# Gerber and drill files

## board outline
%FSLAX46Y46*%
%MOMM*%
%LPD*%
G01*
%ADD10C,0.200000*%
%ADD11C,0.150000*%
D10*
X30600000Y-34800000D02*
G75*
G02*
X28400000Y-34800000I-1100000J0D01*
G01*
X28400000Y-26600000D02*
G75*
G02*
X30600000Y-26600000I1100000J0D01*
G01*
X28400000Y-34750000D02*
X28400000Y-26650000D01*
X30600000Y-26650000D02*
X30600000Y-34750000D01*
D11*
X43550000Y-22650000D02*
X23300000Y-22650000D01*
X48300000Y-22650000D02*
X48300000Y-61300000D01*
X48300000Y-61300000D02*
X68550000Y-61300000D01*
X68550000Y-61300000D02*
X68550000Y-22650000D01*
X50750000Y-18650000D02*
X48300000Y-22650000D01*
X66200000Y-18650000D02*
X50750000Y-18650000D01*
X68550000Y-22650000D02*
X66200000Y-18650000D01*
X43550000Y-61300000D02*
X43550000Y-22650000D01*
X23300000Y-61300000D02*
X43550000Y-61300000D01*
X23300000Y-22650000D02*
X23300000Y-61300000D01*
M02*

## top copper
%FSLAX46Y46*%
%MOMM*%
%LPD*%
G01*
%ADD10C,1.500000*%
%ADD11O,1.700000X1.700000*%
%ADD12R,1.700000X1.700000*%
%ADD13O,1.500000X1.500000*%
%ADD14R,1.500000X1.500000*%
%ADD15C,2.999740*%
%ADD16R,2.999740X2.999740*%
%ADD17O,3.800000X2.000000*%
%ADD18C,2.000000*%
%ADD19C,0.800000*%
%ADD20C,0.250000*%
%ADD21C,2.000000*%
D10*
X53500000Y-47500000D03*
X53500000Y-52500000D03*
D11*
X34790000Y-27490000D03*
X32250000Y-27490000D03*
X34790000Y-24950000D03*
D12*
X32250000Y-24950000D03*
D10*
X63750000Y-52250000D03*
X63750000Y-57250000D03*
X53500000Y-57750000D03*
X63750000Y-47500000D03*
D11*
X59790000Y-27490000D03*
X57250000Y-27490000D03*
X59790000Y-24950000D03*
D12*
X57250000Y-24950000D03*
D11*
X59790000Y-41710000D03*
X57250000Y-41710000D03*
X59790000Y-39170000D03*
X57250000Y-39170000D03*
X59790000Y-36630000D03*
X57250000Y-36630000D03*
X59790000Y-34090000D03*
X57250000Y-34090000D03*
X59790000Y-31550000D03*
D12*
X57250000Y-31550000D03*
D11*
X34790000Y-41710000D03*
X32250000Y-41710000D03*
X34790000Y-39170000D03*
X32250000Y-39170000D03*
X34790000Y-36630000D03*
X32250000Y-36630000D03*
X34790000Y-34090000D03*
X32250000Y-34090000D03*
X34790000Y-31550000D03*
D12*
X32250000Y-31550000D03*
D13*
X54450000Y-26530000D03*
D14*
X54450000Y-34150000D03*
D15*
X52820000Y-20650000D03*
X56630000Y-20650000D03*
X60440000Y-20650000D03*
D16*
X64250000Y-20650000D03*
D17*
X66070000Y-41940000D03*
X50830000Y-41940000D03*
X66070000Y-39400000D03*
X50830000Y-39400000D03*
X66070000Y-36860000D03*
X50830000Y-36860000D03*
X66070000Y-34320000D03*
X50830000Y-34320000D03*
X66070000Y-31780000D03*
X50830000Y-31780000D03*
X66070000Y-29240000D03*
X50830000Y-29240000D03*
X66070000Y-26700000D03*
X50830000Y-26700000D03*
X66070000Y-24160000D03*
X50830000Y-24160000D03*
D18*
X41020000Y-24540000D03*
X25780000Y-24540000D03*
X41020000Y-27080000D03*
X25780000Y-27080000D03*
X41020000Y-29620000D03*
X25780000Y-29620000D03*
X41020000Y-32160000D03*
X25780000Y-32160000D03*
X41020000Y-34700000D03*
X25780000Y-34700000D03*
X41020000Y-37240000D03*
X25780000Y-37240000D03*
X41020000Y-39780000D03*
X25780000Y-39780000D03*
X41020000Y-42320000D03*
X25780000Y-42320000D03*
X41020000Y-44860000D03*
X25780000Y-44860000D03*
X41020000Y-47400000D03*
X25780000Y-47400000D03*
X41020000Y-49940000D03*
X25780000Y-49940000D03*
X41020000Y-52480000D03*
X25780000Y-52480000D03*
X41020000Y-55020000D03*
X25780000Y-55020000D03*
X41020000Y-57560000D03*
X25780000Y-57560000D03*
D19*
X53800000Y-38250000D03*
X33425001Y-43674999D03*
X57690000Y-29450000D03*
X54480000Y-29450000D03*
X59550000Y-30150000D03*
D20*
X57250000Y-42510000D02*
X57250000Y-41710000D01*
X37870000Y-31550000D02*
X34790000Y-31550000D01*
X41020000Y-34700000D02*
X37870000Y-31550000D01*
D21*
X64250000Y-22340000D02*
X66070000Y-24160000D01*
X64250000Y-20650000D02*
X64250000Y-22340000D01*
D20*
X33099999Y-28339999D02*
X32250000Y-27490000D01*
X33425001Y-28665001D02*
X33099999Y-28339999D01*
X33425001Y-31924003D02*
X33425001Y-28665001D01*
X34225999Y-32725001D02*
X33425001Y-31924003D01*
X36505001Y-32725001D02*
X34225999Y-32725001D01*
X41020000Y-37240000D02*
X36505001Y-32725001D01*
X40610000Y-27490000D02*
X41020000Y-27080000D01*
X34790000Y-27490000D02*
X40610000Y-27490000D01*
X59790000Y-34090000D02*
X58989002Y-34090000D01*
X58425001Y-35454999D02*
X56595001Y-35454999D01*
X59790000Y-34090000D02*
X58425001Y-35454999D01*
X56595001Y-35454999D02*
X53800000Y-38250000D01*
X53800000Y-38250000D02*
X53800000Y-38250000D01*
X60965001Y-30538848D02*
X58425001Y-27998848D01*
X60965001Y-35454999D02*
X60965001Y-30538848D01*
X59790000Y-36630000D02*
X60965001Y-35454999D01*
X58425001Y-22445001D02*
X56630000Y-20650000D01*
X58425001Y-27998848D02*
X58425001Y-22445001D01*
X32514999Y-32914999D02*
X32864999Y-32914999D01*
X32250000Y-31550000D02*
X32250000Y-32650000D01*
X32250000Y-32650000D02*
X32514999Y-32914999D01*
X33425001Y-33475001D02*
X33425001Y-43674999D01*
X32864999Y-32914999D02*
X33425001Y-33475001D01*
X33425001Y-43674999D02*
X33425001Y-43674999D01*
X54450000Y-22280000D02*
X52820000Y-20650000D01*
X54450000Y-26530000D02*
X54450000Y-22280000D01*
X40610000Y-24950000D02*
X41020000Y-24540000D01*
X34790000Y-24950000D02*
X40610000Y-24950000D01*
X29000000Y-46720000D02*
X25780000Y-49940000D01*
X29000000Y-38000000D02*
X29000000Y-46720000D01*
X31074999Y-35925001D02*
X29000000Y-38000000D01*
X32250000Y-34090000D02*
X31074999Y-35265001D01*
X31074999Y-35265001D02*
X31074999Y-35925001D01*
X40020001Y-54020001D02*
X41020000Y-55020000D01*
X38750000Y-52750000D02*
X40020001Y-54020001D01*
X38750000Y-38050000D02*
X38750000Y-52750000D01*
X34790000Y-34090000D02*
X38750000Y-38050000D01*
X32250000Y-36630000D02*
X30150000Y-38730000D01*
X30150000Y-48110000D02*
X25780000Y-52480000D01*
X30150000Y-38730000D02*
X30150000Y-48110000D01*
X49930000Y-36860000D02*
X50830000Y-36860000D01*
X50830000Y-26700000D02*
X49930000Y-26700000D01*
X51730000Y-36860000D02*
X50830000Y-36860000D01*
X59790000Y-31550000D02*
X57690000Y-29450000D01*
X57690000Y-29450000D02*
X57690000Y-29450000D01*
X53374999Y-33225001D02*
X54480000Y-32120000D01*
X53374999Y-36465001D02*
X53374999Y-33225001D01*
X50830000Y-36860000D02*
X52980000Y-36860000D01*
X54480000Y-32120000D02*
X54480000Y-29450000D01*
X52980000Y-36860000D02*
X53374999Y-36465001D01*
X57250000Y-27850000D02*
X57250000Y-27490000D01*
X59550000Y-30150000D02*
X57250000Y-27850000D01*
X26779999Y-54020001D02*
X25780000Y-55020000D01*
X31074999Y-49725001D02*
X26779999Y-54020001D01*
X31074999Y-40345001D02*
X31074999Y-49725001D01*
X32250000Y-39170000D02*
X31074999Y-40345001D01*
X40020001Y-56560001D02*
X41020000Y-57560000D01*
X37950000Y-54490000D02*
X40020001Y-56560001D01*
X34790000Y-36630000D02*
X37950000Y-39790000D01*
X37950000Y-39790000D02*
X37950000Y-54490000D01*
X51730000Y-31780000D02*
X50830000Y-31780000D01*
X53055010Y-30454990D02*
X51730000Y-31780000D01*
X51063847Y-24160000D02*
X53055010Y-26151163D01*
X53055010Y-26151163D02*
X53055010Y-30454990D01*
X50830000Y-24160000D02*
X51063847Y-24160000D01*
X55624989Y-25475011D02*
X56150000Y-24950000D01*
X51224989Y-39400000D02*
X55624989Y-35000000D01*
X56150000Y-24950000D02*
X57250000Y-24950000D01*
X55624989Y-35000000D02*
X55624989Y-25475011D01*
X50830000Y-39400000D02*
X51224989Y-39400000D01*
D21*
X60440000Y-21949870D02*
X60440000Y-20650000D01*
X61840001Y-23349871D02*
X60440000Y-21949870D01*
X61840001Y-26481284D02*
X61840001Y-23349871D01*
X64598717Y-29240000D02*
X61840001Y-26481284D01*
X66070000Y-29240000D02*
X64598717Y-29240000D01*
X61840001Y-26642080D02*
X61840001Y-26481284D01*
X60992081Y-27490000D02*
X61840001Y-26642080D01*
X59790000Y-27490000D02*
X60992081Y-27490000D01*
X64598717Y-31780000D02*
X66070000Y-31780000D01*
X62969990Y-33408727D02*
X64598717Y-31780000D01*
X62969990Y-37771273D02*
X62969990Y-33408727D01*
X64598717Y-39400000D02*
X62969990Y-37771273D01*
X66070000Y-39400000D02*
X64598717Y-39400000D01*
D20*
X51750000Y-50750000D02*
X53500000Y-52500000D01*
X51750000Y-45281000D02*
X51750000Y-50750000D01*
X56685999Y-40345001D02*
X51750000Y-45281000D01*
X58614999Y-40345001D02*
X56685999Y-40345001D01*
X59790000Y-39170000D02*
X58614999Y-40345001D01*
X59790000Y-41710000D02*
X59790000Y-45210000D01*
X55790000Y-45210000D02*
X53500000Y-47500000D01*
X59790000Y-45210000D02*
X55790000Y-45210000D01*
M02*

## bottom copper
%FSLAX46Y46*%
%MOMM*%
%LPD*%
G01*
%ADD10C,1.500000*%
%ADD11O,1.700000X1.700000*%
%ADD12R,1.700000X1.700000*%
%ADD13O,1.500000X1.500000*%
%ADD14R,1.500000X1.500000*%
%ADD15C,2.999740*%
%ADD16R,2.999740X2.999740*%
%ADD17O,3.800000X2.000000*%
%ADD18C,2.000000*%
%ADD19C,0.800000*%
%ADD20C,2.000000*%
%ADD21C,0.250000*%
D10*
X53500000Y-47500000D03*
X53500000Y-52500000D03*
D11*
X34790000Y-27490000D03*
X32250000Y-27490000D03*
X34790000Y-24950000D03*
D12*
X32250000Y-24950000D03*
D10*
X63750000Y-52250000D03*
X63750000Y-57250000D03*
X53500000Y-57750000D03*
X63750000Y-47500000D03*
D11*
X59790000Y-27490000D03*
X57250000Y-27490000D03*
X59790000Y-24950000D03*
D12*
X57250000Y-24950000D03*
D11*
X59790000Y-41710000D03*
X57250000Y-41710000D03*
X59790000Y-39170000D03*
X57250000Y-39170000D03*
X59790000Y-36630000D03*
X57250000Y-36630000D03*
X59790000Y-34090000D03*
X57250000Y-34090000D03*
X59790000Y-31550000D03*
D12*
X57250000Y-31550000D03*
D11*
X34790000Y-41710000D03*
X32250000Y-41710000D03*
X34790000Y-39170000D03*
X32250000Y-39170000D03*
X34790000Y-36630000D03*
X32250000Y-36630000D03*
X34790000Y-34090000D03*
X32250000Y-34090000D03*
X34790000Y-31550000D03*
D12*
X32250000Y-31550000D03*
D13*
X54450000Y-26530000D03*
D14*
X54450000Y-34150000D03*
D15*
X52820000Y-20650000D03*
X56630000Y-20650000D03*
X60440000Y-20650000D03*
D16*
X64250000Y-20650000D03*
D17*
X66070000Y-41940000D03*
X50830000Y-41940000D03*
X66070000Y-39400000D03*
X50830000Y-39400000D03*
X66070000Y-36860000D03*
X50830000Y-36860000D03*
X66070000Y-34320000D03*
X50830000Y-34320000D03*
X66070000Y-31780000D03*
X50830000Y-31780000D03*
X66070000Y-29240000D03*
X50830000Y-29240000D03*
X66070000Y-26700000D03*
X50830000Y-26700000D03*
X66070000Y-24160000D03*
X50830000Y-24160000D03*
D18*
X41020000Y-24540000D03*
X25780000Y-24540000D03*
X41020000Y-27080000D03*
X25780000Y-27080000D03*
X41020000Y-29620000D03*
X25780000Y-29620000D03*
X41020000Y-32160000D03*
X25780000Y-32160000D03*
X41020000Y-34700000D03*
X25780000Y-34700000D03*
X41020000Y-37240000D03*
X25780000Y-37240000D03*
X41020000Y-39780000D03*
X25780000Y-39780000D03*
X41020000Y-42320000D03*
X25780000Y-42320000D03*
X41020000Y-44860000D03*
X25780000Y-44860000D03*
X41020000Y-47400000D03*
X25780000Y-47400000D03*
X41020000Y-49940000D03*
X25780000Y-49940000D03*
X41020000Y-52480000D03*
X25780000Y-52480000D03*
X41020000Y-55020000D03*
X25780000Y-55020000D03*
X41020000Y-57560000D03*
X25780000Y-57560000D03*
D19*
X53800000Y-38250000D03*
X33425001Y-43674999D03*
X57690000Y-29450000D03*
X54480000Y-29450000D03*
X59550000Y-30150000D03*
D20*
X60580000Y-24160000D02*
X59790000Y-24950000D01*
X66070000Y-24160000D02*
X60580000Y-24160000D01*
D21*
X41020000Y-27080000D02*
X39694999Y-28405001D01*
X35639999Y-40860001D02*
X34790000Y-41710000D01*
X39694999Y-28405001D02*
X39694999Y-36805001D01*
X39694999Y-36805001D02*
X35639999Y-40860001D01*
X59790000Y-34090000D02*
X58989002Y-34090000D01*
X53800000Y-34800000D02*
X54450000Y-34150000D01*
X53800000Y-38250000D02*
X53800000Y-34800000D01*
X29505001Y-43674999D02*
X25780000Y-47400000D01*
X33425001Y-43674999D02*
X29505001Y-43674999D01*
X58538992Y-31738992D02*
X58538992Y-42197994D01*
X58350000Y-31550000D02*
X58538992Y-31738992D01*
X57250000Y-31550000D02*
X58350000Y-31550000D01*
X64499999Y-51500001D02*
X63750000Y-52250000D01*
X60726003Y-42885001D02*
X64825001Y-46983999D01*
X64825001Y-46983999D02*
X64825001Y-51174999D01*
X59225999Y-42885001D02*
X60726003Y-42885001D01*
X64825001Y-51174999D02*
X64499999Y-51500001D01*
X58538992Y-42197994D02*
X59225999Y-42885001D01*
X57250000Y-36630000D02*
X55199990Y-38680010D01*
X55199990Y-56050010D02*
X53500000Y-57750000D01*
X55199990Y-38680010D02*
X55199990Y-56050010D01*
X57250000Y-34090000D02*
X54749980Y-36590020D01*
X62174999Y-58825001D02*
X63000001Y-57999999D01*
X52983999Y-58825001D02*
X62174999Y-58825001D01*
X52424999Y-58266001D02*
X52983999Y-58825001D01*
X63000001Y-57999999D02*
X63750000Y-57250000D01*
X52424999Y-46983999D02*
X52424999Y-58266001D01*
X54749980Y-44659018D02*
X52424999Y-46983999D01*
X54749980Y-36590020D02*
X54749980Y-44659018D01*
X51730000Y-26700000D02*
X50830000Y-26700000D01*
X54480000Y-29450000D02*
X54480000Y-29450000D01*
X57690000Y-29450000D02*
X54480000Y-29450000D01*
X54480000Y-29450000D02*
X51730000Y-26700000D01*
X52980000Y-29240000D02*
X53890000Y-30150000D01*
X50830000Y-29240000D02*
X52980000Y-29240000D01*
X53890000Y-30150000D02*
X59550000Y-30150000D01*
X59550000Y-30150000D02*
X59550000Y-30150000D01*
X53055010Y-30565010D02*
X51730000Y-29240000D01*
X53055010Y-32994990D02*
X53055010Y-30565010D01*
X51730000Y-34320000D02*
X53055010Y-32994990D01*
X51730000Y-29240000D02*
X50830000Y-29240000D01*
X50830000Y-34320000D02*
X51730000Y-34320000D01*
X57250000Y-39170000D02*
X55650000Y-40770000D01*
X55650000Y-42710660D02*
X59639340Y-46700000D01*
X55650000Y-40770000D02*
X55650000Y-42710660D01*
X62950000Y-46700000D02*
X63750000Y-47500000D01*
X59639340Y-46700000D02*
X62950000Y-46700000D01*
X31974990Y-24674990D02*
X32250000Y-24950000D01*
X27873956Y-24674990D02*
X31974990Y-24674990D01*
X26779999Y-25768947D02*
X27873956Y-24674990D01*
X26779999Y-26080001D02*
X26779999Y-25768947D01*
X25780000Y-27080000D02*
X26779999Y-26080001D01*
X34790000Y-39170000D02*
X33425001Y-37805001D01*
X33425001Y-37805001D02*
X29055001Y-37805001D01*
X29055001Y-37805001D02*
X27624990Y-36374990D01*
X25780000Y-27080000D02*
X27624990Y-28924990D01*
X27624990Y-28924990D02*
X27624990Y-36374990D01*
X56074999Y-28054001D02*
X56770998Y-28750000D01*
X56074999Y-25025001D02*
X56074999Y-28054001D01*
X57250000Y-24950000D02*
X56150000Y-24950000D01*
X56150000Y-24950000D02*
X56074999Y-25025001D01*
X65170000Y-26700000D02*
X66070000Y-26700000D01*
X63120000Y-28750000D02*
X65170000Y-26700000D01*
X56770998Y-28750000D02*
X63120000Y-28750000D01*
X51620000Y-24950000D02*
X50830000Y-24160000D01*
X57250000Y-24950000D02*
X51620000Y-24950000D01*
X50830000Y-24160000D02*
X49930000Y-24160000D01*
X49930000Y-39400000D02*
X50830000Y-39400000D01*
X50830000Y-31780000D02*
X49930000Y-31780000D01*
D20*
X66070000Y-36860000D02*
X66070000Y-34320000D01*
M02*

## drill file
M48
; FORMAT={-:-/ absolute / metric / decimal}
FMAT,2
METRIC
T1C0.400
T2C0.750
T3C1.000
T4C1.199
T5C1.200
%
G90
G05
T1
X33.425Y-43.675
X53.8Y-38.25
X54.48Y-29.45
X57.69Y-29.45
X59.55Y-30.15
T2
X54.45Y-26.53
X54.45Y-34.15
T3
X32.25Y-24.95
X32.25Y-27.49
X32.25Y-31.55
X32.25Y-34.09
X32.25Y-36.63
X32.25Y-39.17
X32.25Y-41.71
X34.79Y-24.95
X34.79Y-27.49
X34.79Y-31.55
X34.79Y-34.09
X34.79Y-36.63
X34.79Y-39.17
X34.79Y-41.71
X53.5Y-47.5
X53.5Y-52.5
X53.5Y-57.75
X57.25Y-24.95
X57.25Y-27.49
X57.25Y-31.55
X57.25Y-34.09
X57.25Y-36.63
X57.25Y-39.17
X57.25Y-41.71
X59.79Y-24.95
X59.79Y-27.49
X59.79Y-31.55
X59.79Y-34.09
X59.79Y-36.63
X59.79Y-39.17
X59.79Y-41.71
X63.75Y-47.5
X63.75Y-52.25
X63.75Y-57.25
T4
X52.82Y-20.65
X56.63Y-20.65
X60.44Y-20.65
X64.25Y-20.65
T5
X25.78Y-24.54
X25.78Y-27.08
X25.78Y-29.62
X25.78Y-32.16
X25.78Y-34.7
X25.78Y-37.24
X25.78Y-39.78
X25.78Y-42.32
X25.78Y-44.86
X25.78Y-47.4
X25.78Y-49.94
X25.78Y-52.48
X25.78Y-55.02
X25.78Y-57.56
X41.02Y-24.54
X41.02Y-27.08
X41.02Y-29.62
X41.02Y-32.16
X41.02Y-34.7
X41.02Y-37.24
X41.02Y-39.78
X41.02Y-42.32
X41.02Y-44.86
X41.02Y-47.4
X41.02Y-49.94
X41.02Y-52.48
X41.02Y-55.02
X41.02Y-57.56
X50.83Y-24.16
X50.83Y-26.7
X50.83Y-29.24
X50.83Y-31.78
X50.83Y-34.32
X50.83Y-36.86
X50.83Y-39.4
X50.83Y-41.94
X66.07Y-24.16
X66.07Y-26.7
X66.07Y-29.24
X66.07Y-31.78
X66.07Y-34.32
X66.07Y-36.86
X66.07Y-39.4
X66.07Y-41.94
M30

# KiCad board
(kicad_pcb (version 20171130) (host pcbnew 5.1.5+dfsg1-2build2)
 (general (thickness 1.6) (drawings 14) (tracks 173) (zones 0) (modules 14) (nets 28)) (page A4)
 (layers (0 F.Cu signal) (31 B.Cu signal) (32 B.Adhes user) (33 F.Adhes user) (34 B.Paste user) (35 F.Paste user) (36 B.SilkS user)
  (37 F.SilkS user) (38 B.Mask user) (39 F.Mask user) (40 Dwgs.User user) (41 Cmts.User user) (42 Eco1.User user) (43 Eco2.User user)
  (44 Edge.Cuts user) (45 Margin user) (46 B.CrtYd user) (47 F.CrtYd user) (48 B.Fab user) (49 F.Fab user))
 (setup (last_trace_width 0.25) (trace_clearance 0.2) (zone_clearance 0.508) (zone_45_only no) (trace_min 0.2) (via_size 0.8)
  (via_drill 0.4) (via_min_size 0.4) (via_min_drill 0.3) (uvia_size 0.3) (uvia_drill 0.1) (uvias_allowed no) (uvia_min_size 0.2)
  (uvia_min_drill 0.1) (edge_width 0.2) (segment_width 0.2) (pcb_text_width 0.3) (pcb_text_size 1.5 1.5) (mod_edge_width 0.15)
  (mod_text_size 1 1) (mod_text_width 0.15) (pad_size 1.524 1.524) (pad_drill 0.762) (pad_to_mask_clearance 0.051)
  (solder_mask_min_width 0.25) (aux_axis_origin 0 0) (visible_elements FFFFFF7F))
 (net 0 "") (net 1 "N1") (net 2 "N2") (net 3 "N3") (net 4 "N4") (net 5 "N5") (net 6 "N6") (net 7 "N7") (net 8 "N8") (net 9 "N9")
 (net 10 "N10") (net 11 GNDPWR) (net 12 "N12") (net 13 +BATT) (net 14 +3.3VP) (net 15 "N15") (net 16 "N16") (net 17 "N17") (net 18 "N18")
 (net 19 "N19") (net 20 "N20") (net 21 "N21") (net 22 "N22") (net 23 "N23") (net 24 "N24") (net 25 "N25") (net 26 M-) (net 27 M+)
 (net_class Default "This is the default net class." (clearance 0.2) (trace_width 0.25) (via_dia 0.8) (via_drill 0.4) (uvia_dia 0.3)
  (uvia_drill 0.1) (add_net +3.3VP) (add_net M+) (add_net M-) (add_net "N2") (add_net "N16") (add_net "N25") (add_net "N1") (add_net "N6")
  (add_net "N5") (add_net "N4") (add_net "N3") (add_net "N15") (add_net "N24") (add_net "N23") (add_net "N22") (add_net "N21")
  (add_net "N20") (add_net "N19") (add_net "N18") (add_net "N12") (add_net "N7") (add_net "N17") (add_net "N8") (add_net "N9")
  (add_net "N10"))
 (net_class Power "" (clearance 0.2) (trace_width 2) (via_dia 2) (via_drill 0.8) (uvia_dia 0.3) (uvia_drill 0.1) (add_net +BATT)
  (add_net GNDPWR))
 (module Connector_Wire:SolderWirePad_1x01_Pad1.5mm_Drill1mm (layer B.Cu) (at 53.5 47.5)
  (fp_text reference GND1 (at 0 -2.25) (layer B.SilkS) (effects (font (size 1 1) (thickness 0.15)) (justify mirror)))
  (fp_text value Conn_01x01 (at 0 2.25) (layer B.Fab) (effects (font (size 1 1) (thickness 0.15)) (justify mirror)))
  (pad 1 thru_hole circle (at 0 0) (size 1.5 1.5) (drill 1) (layers *.Cu *.Mask) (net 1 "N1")))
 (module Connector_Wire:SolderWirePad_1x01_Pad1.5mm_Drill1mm (layer B.Cu) (at 53.5 52.5)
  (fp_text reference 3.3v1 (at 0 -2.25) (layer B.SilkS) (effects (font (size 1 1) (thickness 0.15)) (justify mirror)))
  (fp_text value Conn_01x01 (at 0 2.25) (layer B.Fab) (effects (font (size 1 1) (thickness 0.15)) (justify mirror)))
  (pad 1 thru_hole circle (at 0 0) (size 1.5 1.5) (drill 1) (layers *.Cu *.Mask) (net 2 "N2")))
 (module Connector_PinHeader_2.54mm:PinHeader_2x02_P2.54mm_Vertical (layer F.Cu) (at 32.25 24.95)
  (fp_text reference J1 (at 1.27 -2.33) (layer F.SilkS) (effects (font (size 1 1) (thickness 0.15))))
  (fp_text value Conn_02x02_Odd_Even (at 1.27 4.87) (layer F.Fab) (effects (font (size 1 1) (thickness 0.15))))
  (pad 4 thru_hole oval (at 2.54 2.54) (size 1.7 1.7) (drill 1) (layers *.Cu *.Mask) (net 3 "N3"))
  (pad 3 thru_hole oval (at 0 2.54) (size 1.7 1.7) (drill 1) (layers *.Cu *.Mask) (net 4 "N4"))
  (pad 2 thru_hole oval (at 2.54 0) (size 1.7 1.7) (drill 1) (layers *.Cu *.Mask) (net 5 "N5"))
  (pad 1 thru_hole rect (at 0 0) (size 1.7 1.7) (drill 1) (layers *.Cu *.Mask) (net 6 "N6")))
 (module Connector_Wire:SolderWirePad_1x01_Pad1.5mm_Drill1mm (layer B.Cu) (at 63.75 52.25)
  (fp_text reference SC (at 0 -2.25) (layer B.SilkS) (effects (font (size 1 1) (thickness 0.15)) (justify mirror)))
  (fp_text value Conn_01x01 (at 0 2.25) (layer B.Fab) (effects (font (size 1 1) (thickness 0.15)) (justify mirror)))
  (pad 1 thru_hole circle (at 0 0) (size 1.5 1.5) (drill 1) (layers *.Cu *.Mask) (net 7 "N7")))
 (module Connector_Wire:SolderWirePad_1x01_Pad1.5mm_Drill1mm (layer B.Cu) (at 63.75 57.25)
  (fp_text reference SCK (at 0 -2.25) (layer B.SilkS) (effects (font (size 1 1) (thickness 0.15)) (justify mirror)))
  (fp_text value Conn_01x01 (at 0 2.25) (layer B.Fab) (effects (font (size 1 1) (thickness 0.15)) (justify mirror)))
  (pad 1 thru_hole circle (at 0 0) (size 1.5 1.5) (drill 1) (layers *.Cu *.Mask) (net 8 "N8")))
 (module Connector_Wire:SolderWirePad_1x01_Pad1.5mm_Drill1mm (layer B.Cu) (at 53.5 57.75)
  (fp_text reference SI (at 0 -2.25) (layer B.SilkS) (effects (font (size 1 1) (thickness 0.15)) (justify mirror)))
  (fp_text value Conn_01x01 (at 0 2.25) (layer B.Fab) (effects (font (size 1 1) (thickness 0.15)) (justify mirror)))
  (pad 1 thru_hole circle (at 0 0) (size 1.5 1.5) (drill 1) (layers *.Cu *.Mask) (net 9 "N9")))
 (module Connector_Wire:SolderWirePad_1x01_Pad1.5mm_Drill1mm (layer B.Cu) (at 63.75 47.5)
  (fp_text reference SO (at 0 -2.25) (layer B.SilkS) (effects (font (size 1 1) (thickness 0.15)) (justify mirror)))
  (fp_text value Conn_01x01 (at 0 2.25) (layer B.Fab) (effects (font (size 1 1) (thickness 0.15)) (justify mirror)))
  (pad 1 thru_hole circle (at 0 0) (size 1.5 1.5) (drill 1) (layers *.Cu *.Mask) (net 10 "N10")))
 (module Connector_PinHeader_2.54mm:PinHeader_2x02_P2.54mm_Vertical (layer F.Cu) (at 57.25 24.95)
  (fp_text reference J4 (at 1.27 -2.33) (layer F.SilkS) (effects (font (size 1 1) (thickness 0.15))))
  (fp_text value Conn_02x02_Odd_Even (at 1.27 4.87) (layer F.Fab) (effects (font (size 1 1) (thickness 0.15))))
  (pad 4 thru_hole oval (at 2.54 2.54) (size 1.7 1.7) (drill 1) (layers *.Cu *.Mask) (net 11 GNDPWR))
  (pad 3 thru_hole oval (at 0 2.54) (size 1.7 1.7) (drill 1) (layers *.Cu *.Mask) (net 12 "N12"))
  (pad 2 thru_hole oval (at 2.54 0) (size 1.7 1.7) (drill 1) (layers *.Cu *.Mask) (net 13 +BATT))
  (pad 1 thru_hole rect (at 0 0) (size 1.7 1.7) (drill 1) (layers *.Cu *.Mask) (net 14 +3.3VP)))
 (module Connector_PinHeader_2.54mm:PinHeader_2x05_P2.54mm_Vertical (layer F.Cu) (at 57.25 31.55)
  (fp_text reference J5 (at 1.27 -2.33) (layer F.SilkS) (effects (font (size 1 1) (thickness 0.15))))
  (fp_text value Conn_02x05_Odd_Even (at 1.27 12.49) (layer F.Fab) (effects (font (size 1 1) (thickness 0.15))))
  (pad 10 thru_hole oval (at 2.54 10.16) (size 1.7 1.7) (drill 1) (layers *.Cu *.Mask) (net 1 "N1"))
  (pad 9 thru_hole oval (at 0 10.16) (size 1.7 1.7) (drill 1) (layers *.Cu *.Mask))
  (pad 8 thru_hole oval (at 2.54 7.62) (size 1.7 1.7) (drill 1) (layers *.Cu *.Mask) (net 2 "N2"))
  (pad 7 thru_hole oval (at 0 7.62) (size 1.7 1.7) (drill 1) (layers *.Cu *.Mask) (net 10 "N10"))
  (pad 6 thru_hole oval (at 2.54 5.08) (size 1.7 1.7) (drill 1) (layers *.Cu *.Mask) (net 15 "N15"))
  (pad 5 thru_hole oval (at 0 5.08) (size 1.7 1.7) (drill 1) (layers *.Cu *.Mask) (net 9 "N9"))
  (pad 4 thru_hole oval (at 2.54 2.54) (size 1.7 1.7) (drill 1) (layers *.Cu *.Mask) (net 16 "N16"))
  (pad 3 thru_hole oval (at 0 2.54) (size 1.7 1.7) (drill 1) (layers *.Cu *.Mask) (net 8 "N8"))
  (pad 2 thru_hole oval (at 2.54 0) (size 1.7 1.7) (drill 1) (layers *.Cu *.Mask) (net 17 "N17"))
  (pad 1 thru_hole rect (at 0 0) (size 1.7 1.7) (drill 1) (layers *.Cu *.Mask) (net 7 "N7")))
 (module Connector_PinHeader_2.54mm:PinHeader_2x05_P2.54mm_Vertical (layer F.Cu) (at 32.25 31.55)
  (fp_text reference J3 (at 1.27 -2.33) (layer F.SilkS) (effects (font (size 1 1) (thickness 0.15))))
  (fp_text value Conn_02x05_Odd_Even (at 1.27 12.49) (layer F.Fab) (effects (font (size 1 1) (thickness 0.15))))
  (pad 10 thru_hole oval (at 2.54 10.16) (size 1.7 1.7) (drill 1) (layers *.Cu *.Mask) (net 3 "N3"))
  (pad 9 thru_hole oval (at 0 10.16) (size 1.7 1.7) (drill 1) (layers *.Cu *.Mask))
  (pad 8 thru_hole oval (at 2.54 7.62) (size 1.7 1.7) (drill 1) (layers *.Cu *.Mask) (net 6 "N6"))
  (pad 7 thru_hole oval (at 0 7.62) (size 1.7 1.7) (drill 1) (layers *.Cu *.Mask) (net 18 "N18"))
  (pad 6 thru_hole oval (at 2.54 5.08) (size 1.7 1.7) (drill 1) (layers *.Cu *.Mask) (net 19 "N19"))
  (pad 5 thru_hole oval (at 0 5.08) (size 1.7 1.7) (drill 1) (layers *.Cu *.Mask) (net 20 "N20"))
  (pad 4 thru_hole oval (at 2.54 2.54) (size 1.7 1.7) (drill 1) (layers *.Cu *.Mask) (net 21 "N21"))
  (pad 3 thru_hole oval (at 0 2.54) (size 1.7 1.7) (drill 1) (layers *.Cu *.Mask) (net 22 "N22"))
  (pad 2 thru_hole oval (at 2.54 0) (size 1.7 1.7) (drill 1) (layers *.Cu *.Mask) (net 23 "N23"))
  (pad 1 thru_hole rect (at 0 0) (size 1.7 1.7) (drill 1) (layers *.Cu *.Mask) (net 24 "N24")))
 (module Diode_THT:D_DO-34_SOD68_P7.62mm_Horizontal (layer F.Cu) (at 54.45 34.15 90)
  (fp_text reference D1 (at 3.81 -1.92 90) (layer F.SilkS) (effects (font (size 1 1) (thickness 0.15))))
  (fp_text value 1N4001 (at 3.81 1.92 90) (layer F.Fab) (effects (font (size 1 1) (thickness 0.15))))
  (pad 2 thru_hole oval (at 7.62 0 90) (size 1.5 1.5) (drill 0.75) (layers *.Cu *.Mask) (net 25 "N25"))
  (pad 1 thru_hole rect (at 0 0 90) (size 1.5 1.5) (drill 0.75) (layers *.Cu *.Mask) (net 16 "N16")))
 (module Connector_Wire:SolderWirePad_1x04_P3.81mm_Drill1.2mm (layer F.Cu) (at 64.25 20.65 180)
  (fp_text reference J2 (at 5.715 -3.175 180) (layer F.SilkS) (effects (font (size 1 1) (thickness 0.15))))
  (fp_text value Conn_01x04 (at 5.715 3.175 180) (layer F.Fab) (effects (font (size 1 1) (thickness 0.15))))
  (pad 4 thru_hole circle (at 11.43 0 180) (size 2.99974 2.99974) (drill 1.19888) (layers *.Cu *.Mask) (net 25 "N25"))
  (pad 3 thru_hole circle (at 7.62 0 180) (size 2.99974 2.99974) (drill 1.19888) (layers *.Cu *.Mask) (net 15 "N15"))
  (pad 2 thru_hole circle (at 3.81 0 180) (size 2.99974 2.99974) (drill 1.19888) (layers *.Cu *.Mask) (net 11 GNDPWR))
  (pad 1 thru_hole rect (at 0 0 180) (size 2.99974 2.99974) (drill 1.19888) (layers *.Cu *.Mask) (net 13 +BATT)))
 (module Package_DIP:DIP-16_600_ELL (layer B.Cu) (at 58.45 33.05 270)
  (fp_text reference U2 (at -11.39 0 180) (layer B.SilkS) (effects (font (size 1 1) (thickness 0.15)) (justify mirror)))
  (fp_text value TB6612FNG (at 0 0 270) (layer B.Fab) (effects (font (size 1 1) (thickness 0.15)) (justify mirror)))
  (pad 8 thru_hole oval (at 8.89 -7.62 270) (size 2 3.8) (drill 1.2) (layers *.Cu *.Mask))
  (pad 9 thru_hole oval (at 8.89 7.62 270) (size 2 3.8) (drill 1.2) (layers *.Cu *.Mask))
  (pad 7 thru_hole oval (at 6.35 -7.62 270) (size 2 3.8) (drill 1.2) (layers *.Cu *.Mask) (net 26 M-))
  (pad 10 thru_hole oval (at 6.35 7.62 270) (size 2 3.8) (drill 1.2) (layers *.Cu *.Mask) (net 14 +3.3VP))
  (pad 6 thru_hole oval (at 3.81 -7.62 270) (size 2 3.8) (drill 1.2) (layers *.Cu *.Mask) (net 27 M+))
  (pad 11 thru_hole oval (at 3.81 7.62 270) (size 2 3.8) (drill 1.2) (layers *.Cu *.Mask) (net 17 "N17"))
  (pad 5 thru_hole oval (at 1.27 -7.62 270) (size 2 3.8) (drill 1.2) (layers *.Cu *.Mask) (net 27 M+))
  (pad 12 thru_hole oval (at 1.27 7.62 270) (size 2 3.8) (drill 1.2) (layers *.Cu *.Mask) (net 12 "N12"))
  (pad 4 thru_hole oval (at -1.27 -7.62 270) (size 2 3.8) (drill 1.2) (layers *.Cu *.Mask) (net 26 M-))
  (pad 13 thru_hole oval (at -1.27 7.62 270) (size 2 3.8) (drill 1.2) (layers *.Cu *.Mask) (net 14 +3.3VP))
  (pad 3 thru_hole oval (at -3.81 -7.62 270) (size 2 3.8) (drill 1.2) (layers *.Cu *.Mask) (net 11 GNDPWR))
  (pad 14 thru_hole oval (at -3.81 7.62 270) (size 2 3.8) (drill 1.2) (layers *.Cu *.Mask) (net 12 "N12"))
  (pad 2 thru_hole oval (at -6.35 -7.62 270) (size 2 3.8) (drill 1.2) (layers *.Cu *.Mask) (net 14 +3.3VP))
  (pad 15 thru_hole oval (at -6.35 7.62 270) (size 2 3.8) (drill 1.2) (layers *.Cu *.Mask) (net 17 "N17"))
  (pad 1 thru_hole oval (at -8.89 -7.62 270) (size 2 3.8) (drill 1.2) (layers *.Cu *.Mask) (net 13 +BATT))
  (pad 16 thru_hole oval (at -8.89 7.62 270) (size 2 3.8) (drill 1.2) (layers *.Cu *.Mask) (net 14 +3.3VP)))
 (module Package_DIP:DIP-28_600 (layer F.Cu) (at 33.4 41.05 270)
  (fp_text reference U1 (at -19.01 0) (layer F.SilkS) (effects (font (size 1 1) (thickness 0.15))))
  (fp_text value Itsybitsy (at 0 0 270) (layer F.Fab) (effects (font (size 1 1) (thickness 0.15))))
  (pad 28 thru_hole circle (at -16.51 -7.62 270) (size 2 2) (drill 1.2) (layers *.Cu *.Mask) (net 5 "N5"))
  (pad 1 thru_hole circle (at -16.51 7.62 270) (size 2 2) (drill 1.2) (layers *.Cu *.Mask))
  (pad 27 thru_hole circle (at -13.97 -7.62 270) (size 2 2) (drill 1.2) (layers *.Cu *.Mask) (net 3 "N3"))
  (pad 2 thru_hole circle (at -13.97 7.62 270) (size 2 2) (drill 1.2) (layers *.Cu *.Mask) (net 6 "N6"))
  (pad 26 thru_hole circle (at -11.43 -7.62 270) (size 2 2) (drill 1.2) (layers *.Cu *.Mask))
  (pad 3 thru_hole circle (at -11.43 7.62 270) (size 2 2) (drill 1.2) (layers *.Cu *.Mask))
  (pad 25 thru_hole circle (at -8.89 -7.62 270) (size 2 2) (drill 1.2) (layers *.Cu *.Mask))
  (pad 4 thru_hole circle (at -8.89 7.62 270) (size 2 2) (drill 1.2) (layers *.Cu *.Mask))
  (pad 24 thru_hole circle (at -6.35 -7.62 270) (size 2 2) (drill 1.2) (layers *.Cu *.Mask) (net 23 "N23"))
  (pad 5 thru_hole circle (at -6.35 7.62 270) (size 2 2) (drill 1.2) (layers *.Cu *.Mask))
  (pad 23 thru_hole circle (at -3.81 -7.62 270) (size 2 2) (drill 1.2) (layers *.Cu *.Mask) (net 4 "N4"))
  (pad 6 thru_hole circle (at -3.81 7.62 270) (size 2 2) (drill 1.2) (layers *.Cu *.Mask))
  (pad 22 thru_hole circle (at -1.27 -7.62 270) (size 2 2) (drill 1.2) (layers *.Cu *.Mask))
  (pad 7 thru_hole circle (at -1.27 7.62 270) (size 2 2) (drill 1.2) (layers *.Cu *.Mask))
  (pad 21 thru_hole circle (at 1.27 -7.62 270) (size 2 2) (drill 1.2) (layers *.Cu *.Mask))
  (pad 8 thru_hole circle (at 1.27 7.62 270) (size 2 2) (drill 1.2) (layers *.Cu *.Mask))
  (pad 20 thru_hole circle (at 3.81 -7.62 270) (size 2 2) (drill 1.2) (layers *.Cu *.Mask))
  (pad 9 thru_hole circle (at 3.81 7.62 270) (size 2 2) (drill 1.2) (layers *.Cu *.Mask))
  (pad 19 thru_hole circle (at 6.35 -7.62 270) (size 2 2) (drill 1.2) (layers *.Cu *.Mask))
  (pad 10 thru_hole circle (at 6.35 7.62 270) (size 2 2) (drill 1.2) (layers *.Cu *.Mask) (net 24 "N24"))
  (pad 18 thru_hole circle (at 8.89 -7.62 270) (size 2 2) (drill 1.2) (layers *.Cu *.Mask))
  (pad 11 thru_hole circle (at 8.89 7.62 270) (size 2 2) (drill 1.2) (layers *.Cu *.Mask) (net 22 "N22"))
  (pad 17 thru_hole circle (at 11.43 -7.62 270) (size 2 2) (drill 1.2) (layers *.Cu *.Mask))
  (pad 12 thru_hole circle (at 11.43 7.62 270) (size 2 2) (drill 1.2) (layers *.Cu *.Mask) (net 20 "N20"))
  (pad 16 thru_hole circle (at 13.97 -7.62 270) (size 2 2) (drill 1.2) (layers *.Cu *.Mask) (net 21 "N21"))
  (pad 13 thru_hole circle (at 13.97 7.62 270) (size 2 2) (drill 1.2) (layers *.Cu *.Mask) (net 18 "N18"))
  (pad 15 thru_hole circle (at 16.51 -7.62 270) (size 2 2) (drill 1.2) (layers *.Cu *.Mask) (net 19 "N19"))
  (pad 14 thru_hole circle (at 16.51 7.62 270) (size 2 2) (drill 1.2) (layers *.Cu *.Mask)))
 (gr_arc (start 29.5 34.8) (end 28.4 34.8) (angle -180) (layer Edge.Cuts) (width 0.2))
 (gr_arc (start 29.5 26.6) (end 30.6 26.6) (angle -180) (layer Edge.Cuts) (width 0.2))
 (gr_line (start 28.4 34.75) (end 28.4 26.65) (layer Edge.Cuts) (width 0.2))
 (gr_line (start 30.6 26.65) (end 30.6 34.75) (layer Edge.Cuts) (width 0.2))
 (gr_line (start 43.55 22.65) (end 23.3 22.65) (layer Edge.Cuts) (width 0.15))
 (gr_line (start 48.3 22.65) (end 48.3 61.3) (layer Edge.Cuts) (width 0.15))
 (gr_line (start 48.3 61.3) (end 68.55 61.3) (layer Edge.Cuts) (width 0.15))
 (gr_line (start 68.55 61.3) (end 68.55 22.65) (layer Edge.Cuts) (width 0.15))
 (gr_line (start 50.75 18.65) (end 48.3 22.65) (layer Edge.Cuts) (width 0.15))
 (gr_line (start 66.2 18.65) (end 50.75 18.65) (layer Edge.Cuts) (width 0.15))
 (gr_line (start 68.55 22.65) (end 66.2 18.65) (layer Edge.Cuts) (width 0.15))
 (gr_line (start 43.55 61.3) (end 43.55 22.65) (layer Edge.Cuts) (width 0.15))
 (gr_line (start 23.3 61.3) (end 43.55 61.3) (layer Edge.Cuts) (width 0.15))
 (gr_line (start 23.3 22.65) (end 23.3 61.3) (layer Edge.Cuts) (width 0.15))
 (segment (start 57.25 42.51) (end 57.25 41.71) (width 0.25) (layer F.Cu) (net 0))
 (segment (start 37.87 31.55) (end 34.79 31.55) (width 0.25) (layer F.Cu) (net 23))
 (segment (start 41.02 34.7) (end 37.87 31.55) (width 0.25) (layer F.Cu) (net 23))
 (segment (start 60.58 24.16) (end 59.79 24.95) (width 2) (layer B.Cu) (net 13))
 (segment (start 66.07 24.16) (end 60.58 24.16) (width 2) (layer B.Cu) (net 13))
 (segment (start 64.25 22.34) (end 66.07 24.16) (width 2) (layer F.Cu) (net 13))
 (segment (start 64.25 20.65) (end 64.25 22.34) (width 2) (layer F.Cu) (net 13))
 (segment (start 33.099999 28.339999) (end 32.25 27.49) (width 0.25) (layer F.Cu) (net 4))
 (segment (start 33.425001 28.665001) (end 33.099999 28.339999) (width 0.25) (layer F.Cu) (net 4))
 (segment (start 33.425001 31.924003) (end 33.425001 28.665001) (width 0.25) (layer F.Cu) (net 4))
 (segment (start 34.225999 32.725001) (end 33.425001 31.924003) (width 0.25) (layer F.Cu) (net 4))
 (segment (start 36.505001 32.725001) (end 34.225999 32.725001) (width 0.25) (layer F.Cu) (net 4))
 (segment (start 41.02 37.24) (end 36.505001 32.725001) (width 0.25) (layer F.Cu) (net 4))
 (segment (start 40.61 27.49) (end 41.02 27.08) (width 0.25) (layer F.Cu) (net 3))
 (segment (start 34.79 27.49) (end 40.61 27.49) (width 0.25) (layer F.Cu) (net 3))
 (segment (start 41.02 27.08) (end 39.694999 28.405001) (width 0.25) (layer B.Cu) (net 3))
 (segment (start 35.639999 40.860001) (end 34.79 41.71) (width 0.25) (layer B.Cu) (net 3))
 (segment (start 39.694999 28.405001) (end 39.694999 36.805001) (width 0.25) (layer B.Cu) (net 3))
 (segment (start 39.694999 36.805001) (end 35.639999 40.860001) (width 0.25) (layer B.Cu) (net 3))
 (segment (start 59.79 34.09) (end 58.989002 34.09) (width 0.25) (layer F.Cu) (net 16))
 (segment (start 59.79 34.09) (end 58.989002 34.09) (width 0.25) (layer B.Cu) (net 16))
 (segment (start 58.425001 35.454999) (end 56.595001 35.454999) (width 0.25) (layer F.Cu) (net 16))
 (segment (start 59.79 34.09) (end 58.425001 35.454999) (width 0.25) (layer F.Cu) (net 16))
 (segment (start 56.595001 35.454999) (end 53.8 38.25) (width 0.25) (layer F.Cu) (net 16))
 (segment (start 53.8 38.25) (end 53.8 38.25) (width 0.25) (layer F.Cu) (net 16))
 (via (at 53.8 38.25) (size 0.8) (drill 0.4) (layers F.Cu B.Cu) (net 16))
 (segment (start 53.8 34.8) (end 54.45 34.15) (width 0.25) (layer B.Cu) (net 16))
 (segment (start 53.8 38.25) (end 53.8 34.8) (width 0.25) (layer B.Cu) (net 16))
 (segment (start 60.965001 30.538848) (end 58.425001 27.998848) (width 0.25) (layer F.Cu) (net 15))
 (segment (start 60.965001 35.454999) (end 60.965001 30.538848) (width 0.25) (layer F.Cu) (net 15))
 (segment (start 59.79 36.63) (end 60.965001 35.454999) (width 0.25) (layer F.Cu) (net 15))
 (segment (start 58.425001 22.445001) (end 56.63 20.65) (width 0.25) (layer F.Cu) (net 15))
 (segment (start 58.425001 27.998848) (end 58.425001 22.445001) (width 0.25) (layer F.Cu) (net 15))
 (segment (start 32.514999 32.914999) (end 32.864999 32.914999) (width 0.25) (layer F.Cu) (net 24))
 (segment (start 32.25 31.55) (end 32.25 32.65) (width 0.25) (layer F.Cu) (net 24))
 (segment (start 32.25 32.65) (end 32.514999 32.914999) (width 0.25) (layer F.Cu) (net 24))
 (segment (start 33.425001 33.475001) (end 33.425001 43.674999) (width 0.25) (layer F.Cu) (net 24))
 (segment (start 32.864999 32.914999) (end 33.425001 33.475001) (width 0.25) (layer F.Cu) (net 24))
 (segment (start 33.425001 43.674999) (end 33.425001 43.674999) (width 0.25) (layer F.Cu) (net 24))
 (via (at 33.425001 43.674999) (size 0.8) (drill 0.4) (layers F.Cu B.Cu) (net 24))
 (segment (start 29.505001 43.674999) (end 25.78 47.4) (width 0.25) (layer B.Cu) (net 24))
 (segment (start 33.425001 43.674999) (end 29.505001 43.674999) (width 0.25) (layer B.Cu) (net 24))
 (segment (start 54.45 22.28) (end 52.82 20.65) (width 0.25) (layer F.Cu) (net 25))
 (segment (start 54.45 26.53) (end 54.45 22.28) (width 0.25) (layer F.Cu) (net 25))
 (segment (start 40.61 24.95) (end 41.02 24.54) (width 0.25) (layer F.Cu) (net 5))
 (segment (start 34.79 24.95) (end 40.61 24.95) (width 0.25) (layer F.Cu) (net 5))
 (segment (start 29 46.72) (end 25.78 49.94) (width 0.25) (layer F.Cu) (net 22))
 (segment (start 29 38) (end 29 46.72) (width 0.25) (layer F.Cu) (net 22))
 (segment (start 31.074999 35.925001) (end 29 38) (width 0.25) (layer F.Cu) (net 22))
 (segment (start 32.25 34.09) (end 31.074999 35.265001) (width 0.25) (layer F.Cu) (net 22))
 (segment (start 31.074999 35.265001) (end 31.074999 35.925001) (width 0.25) (layer F.Cu) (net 22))
 (segment (start 40.020001 54.020001) (end 41.02 55.02) (width 0.25) (layer F.Cu) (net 21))
 (segment (start 38.75 52.75) (end 40.020001 54.020001) (width 0.25) (layer F.Cu) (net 21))
 (segment (start 38.75 38.05) (end 38.75 52.75) (width 0.25) (layer F.Cu) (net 21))
 (segment (start 34.79 34.09) (end 38.75 38.05) (width 0.25) (layer F.Cu) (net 21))
 (segment (start 32.25 36.63) (end 30.15 38.73) (width 0.25) (layer F.Cu) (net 20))
 (segment (start 30.15 48.11) (end 25.78 52.48) (width 0.25) (layer F.Cu) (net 20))
 (segment (start 30.15 38.73) (end 30.15 48.11) (width 0.25) (layer F.Cu) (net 20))
 (segment (start 58.538992 31.738992) (end 58.538992 42.197994) (width 0.25) (layer B.Cu) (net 7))
 (segment (start 58.35 31.55) (end 58.538992 31.738992) (width 0.25) (layer B.Cu) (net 7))
 (segment (start 57.25 31.55) (end 58.35 31.55) (width 0.25) (layer B.Cu) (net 7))
 (segment (start 64.499999 51.500001) (end 63.75 52.25) (width 0.25) (layer B.Cu) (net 7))
 (segment (start 60.726003 42.885001) (end 64.825001 46.983999) (width 0.25) (layer B.Cu) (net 7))
 (segment (start 64.825001 46.983999) (end 64.825001 51.174999) (width 0.25) (layer B.Cu) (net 7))
 (segment (start 59.225999 42.885001) (end 60.726003 42.885001) (width 0.25) (layer B.Cu) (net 7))
 (segment (start 64.825001 51.174999) (end 64.499999 51.500001) (width 0.25) (layer B.Cu) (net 7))
 (segment (start 58.538992 42.197994) (end 59.225999 42.885001) (width 0.25) (layer B.Cu) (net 7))
 (segment (start 57.25 36.63) (end 55.19999 38.68001) (width 0.25) (layer B.Cu) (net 9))
 (segment (start 55.19999 56.05001) (end 53.5 57.75) (width 0.25) (layer B.Cu) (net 9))
 (segment (start 55.19999 38.68001) (end 55.19999 56.05001) (width 0.25) (layer B.Cu) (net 9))
 (segment (start 57.25 34.09) (end 54.74998 36.59002) (width 0.25) (layer B.Cu) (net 8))
 (segment (start 62.174999 58.825001) (end 63.000001 57.999999) (width 0.25) (layer B.Cu) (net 8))
 (segment (start 52.983999 58.825001) (end 62.174999 58.825001) (width 0.25) (layer B.Cu) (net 8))
 (segment (start 52.424999 58.266001) (end 52.983999 58.825001) (width 0.25) (layer B.Cu) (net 8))
 (segment (start 63.000001 57.999999) (end 63.75 57.25) (width 0.25) (layer B.Cu) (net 8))
 (segment (start 52.424999 46.983999) (end 52.424999 58.266001) (width 0.25) (layer B.Cu) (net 8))
 (segment (start 54.74998 44.659018) (end 52.424999 46.983999) (width 0.25) (layer B.Cu) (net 8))
 (segment (start 54.74998 36.59002) (end 54.74998 44.659018) (width 0.25) (layer B.Cu) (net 8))
 (segment (start 49.93 36.86) (end 50.83 36.86) (width 0.25) (layer F.Cu) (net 17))
 (segment (start 50.83 26.7) (end 49.93 26.7) (width 0.25) (layer F.Cu) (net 17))
 (segment (start 51.73 36.86) (end 50.83 36.86) (width 0.25) (layer F.Cu) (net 17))
 (segment (start 59.79 31.55) (end 57.69 29.45) (width 0.25) (layer F.Cu) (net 17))
 (segment (start 57.69 29.45) (end 57.69 29.45) (width 0.25) (layer F.Cu) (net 17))
 (via (at 57.69 29.45) (size 0.8) (drill 0.4) (layers F.Cu B.Cu) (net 17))
 (segment (start 51.73 26.7) (end 50.83 26.7) (width 0.25) (layer B.Cu) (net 17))
 (segment (start 54.48 29.45) (end 54.48 29.45) (width 0.25) (layer B.Cu) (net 17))
 (segment (start 57.69 29.45) (end 54.48 29.45) (width 0.25) (layer B.Cu) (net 17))
 (segment (start 54.48 29.45) (end 51.73 26.7) (width 0.25) (layer B.Cu) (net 17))
 (via (at 54.48 29.45) (size 0.8) (drill 0.4) (layers F.Cu B.Cu) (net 17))
 (segment (start 53.374999 33.225001) (end 54.48 32.12) (width 0.25) (layer F.Cu) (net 17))
 (segment (start 53.374999 36.465001) (end 53.374999 33.225001) (width 0.25) (layer F.Cu) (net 17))
 (segment (start 50.83 36.86) (end 52.98 36.86) (width 0.25) (layer F.Cu) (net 17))
 (segment (start 54.48 32.12) (end 54.48 29.45) (width 0.25) (layer F.Cu) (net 17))
 (segment (start 52.98 36.86) (end 53.374999 36.465001) (width 0.25) (layer F.Cu) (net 17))
 (segment (start 52.98 29.24) (end 53.89 30.15) (width 0.25) (layer B.Cu) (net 12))
 (segment (start 50.83 29.24) (end 52.98 29.24) (width 0.25) (layer B.Cu) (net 12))
 (segment (start 53.89 30.15) (end 59.55 30.15) (width 0.25) (layer B.Cu) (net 12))
 (segment (start 59.55 30.15) (end 59.55 30.15) (width 0.25) (layer B.Cu) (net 12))
 (via (at 59.55 30.15) (size 0.8) (drill 0.4) (layers F.Cu B.Cu) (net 12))
 (segment (start 57.25 27.85) (end 57.25 27.49) (width 0.25) (layer F.Cu) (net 12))
 (segment (start 59.55 30.15) (end 57.25 27.85) (width 0.25) (layer F.Cu) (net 12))
 (segment (start 53.05501 30.56501) (end 51.73 29.24) (width 0.25) (layer B.Cu) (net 12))
 (segment (start 53.05501 32.99499) (end 53.05501 30.56501) (width 0.25) (layer B.Cu) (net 12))
 (segment (start 51.73 34.32) (end 53.05501 32.99499) (width 0.25) (layer B.Cu) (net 12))
 (segment (start 51.73 29.24) (end 50.83 29.24) (width 0.25) (layer B.Cu) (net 12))
 (segment (start 50.83 34.32) (end 51.73 34.32) (width 0.25) (layer B.Cu) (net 12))
 (segment (start 26.779999 54.020001) (end 25.78 55.02) (width 0.25) (layer F.Cu) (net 18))
 (segment (start 31.074999 49.725001) (end 26.779999 54.020001) (width 0.25) (layer F.Cu) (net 18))
 (segment (start 31.074999 40.345001) (end 31.074999 49.725001) (width 0.25) (layer F.Cu) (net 18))
 (segment (start 32.25 39.17) (end 31.074999 40.345001) (width 0.25) (layer F.Cu) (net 18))
 (segment (start 40.020001 56.560001) (end 41.02 57.56) (width 0.25) (layer F.Cu) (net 19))
 (segment (start 37.95 54.49) (end 40.020001 56.560001) (width 0.25) (layer F.Cu) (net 19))
 (segment (start 34.79 36.63) (end 37.95 39.79) (width 0.25) (layer F.Cu) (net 19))
 (segment (start 37.95 39.79) (end 37.95 54.49) (width 0.25) (layer F.Cu) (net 19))
 (segment (start 57.25 39.17) (end 55.65 40.77) (width 0.25) (layer B.Cu) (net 10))
 (segment (start 55.65 42.71066) (end 59.63934 46.7) (width 0.25) (layer B.Cu) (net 10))
 (segment (start 55.65 40.77) (end 55.65 42.71066) (width 0.25) (layer B.Cu) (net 10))
 (segment (start 62.95 46.7) (end 63.75 47.5) (width 0.25) (layer B.Cu) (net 10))
 (segment (start 59.63934 46.7) (end 62.95 46.7) (width 0.25) (layer B.Cu) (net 10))
 (segment (start 31.97499 24.67499) (end 32.25 24.95) (width 0.25) (layer B.Cu) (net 6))
 (segment (start 27.873956 24.67499) (end 31.97499 24.67499) (width 0.25) (layer B.Cu) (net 6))
 (segment (start 26.779999 25.768947) (end 27.873956 24.67499) (width 0.25) (layer B.Cu) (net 6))
 (segment (start 26.779999 26.080001) (end 26.779999 25.768947) (width 0.25) (layer B.Cu) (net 6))
 (segment (start 25.78 27.08) (end 26.779999 26.080001) (width 0.25) (layer B.Cu) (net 6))
 (segment (start 34.79 39.17) (end 33.425001 37.805001) (width 0.25) (layer B.Cu) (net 6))
 (segment (start 33.425001 37.805001) (end 29.055001 37.805001) (width 0.25) (layer B.Cu) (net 6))
 (segment (start 29.055001 37.805001) (end 27.62499 36.37499) (width 0.25) (layer B.Cu) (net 6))
 (segment (start 25.78 27.08) (end 27.62499 28.92499) (width 0.25) (layer B.Cu) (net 6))
 (segment (start 27.62499 28.92499) (end 27.62499 36.37499) (width 0.25) (layer B.Cu) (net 6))
 (segment (start 56.074999 28.054001) (end 56.770998 28.75) (width 0.25) (layer B.Cu) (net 14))
 (segment (start 56.074999 25.025001) (end 56.074999 28.054001) (width 0.25) (layer B.Cu) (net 14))
 (segment (start 57.25 24.95) (end 56.15 24.95) (width 0.25) (layer B.Cu) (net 14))
 (segment (start 56.15 24.95) (end 56.074999 25.025001) (width 0.25) (layer B.Cu) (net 14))
 (segment (start 65.17 26.7) (end 66.07 26.7) (width 0.25) (layer B.Cu) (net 14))
 (segment (start 63.12 28.75) (end 65.17 26.7) (width 0.25) (layer B.Cu) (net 14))
 (segment (start 56.770998 28.75) (end 63.12 28.75) (width 0.25) (layer B.Cu) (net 14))
 (segment (start 51.62 24.95) (end 50.83 24.16) (width 0.25) (layer B.Cu) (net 14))
 (segment (start 57.25 24.95) (end 51.62 24.95) (width 0.25) (layer B.Cu) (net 14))
 (segment (start 50.83 24.16) (end 49.93 24.16) (width 0.25) (layer B.Cu) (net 14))
 (segment (start 49.93 39.4) (end 50.83 39.4) (width 0.25) (layer B.Cu) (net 14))
 (segment (start 50.83 31.78) (end 49.93 31.78) (width 0.25) (layer B.Cu) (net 14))
 (segment (start 51.73 31.78) (end 50.83 31.78) (width 0.25) (layer F.Cu) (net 14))
 (segment (start 53.05501 30.45499) (end 51.73 31.78) (width 0.25) (layer F.Cu) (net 14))
 (segment (start 51.063847 24.16) (end 53.05501 26.151163) (width 0.25) (layer F.Cu) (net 14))
 (segment (start 53.05501 26.151163) (end 53.05501 30.45499) (width 0.25) (layer F.Cu) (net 14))
 (segment (start 50.83 24.16) (end 51.063847 24.16) (width 0.25) (layer F.Cu) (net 14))
 (segment (start 55.624989 25.475011) (end 56.15 24.95) (width 0.25) (layer F.Cu) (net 14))
 (segment (start 51.224989 39.4) (end 55.624989 35) (width 0.25) (layer F.Cu) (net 14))
 (segment (start 56.15 24.95) (end 57.25 24.95) (width 0.25) (layer F.Cu) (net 14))
 (segment (start 55.624989 35) (end 55.624989 25.475011) (width 0.25) (layer F.Cu) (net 14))
 (segment (start 50.83 39.4) (end 51.224989 39.4) (width 0.25) (layer F.Cu) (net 14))
 (segment (start 60.44 21.94987) (end 60.44 20.65) (width 2) (layer F.Cu) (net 11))
 (segment (start 61.840001 23.349871) (end 60.44 21.94987) (width 2) (layer F.Cu) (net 11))
 (segment (start 61.840001 26.481284) (end 61.840001 23.349871) (width 2) (layer F.Cu) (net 11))
 (segment (start 64.598717 29.24) (end 61.840001 26.481284) (width 2) (layer F.Cu) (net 11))
 (segment (start 66.07 29.24) (end 64.598717 29.24) (width 2) (layer F.Cu) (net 11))
 (segment (start 61.840001 26.64208) (end 61.840001 26.481284) (width 2) (layer F.Cu) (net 11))
 (segment (start 60.992081 27.49) (end 61.840001 26.64208) (width 2) (layer F.Cu) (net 11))
 (segment (start 59.79 27.49) (end 60.992081 27.49) (width 2) (layer F.Cu) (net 11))
 (segment (start 64.598717 31.78) (end 66.07 31.78) (width 2) (layer F.Cu) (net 26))
 (segment (start 62.96999 33.408727) (end 64.598717 31.78) (width 2) (layer F.Cu) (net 26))
 (segment (start 62.96999 37.771273) (end 62.96999 33.408727) (width 2) (layer F.Cu) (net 26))
 (segment (start 64.598717 39.4) (end 62.96999 37.771273) (width 2) (layer F.Cu) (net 26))
 (segment (start 66.07 39.4) (end 64.598717 39.4) (width 2) (layer F.Cu) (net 26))
 (segment (start 66.07 36.86) (end 66.07 34.32) (width 2) (layer B.Cu) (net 27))
 (segment (start 51.75 50.75) (end 53.5 52.5) (width 0.25) (layer F.Cu) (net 2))
 (segment (start 51.75 45.281) (end 51.75 50.75) (width 0.25) (layer F.Cu) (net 2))
 (segment (start 56.685999 40.345001) (end 51.75 45.281) (width 0.25) (layer F.Cu) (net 2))
 (segment (start 58.614999 40.345001) (end 56.685999 40.345001) (width 0.25) (layer F.Cu) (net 2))
 (segment (start 59.79 39.17) (end 58.614999 40.345001) (width 0.25) (layer F.Cu) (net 2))
 (segment (start 59.79 41.71) (end 59.79 45.21) (width 0.25) (layer F.Cu) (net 1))
 (segment (start 55.79 45.21) (end 53.5 47.5) (width 0.25) (layer F.Cu) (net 1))
 (segment (start 59.79 45.21) (end 55.79 45.21) (width 0.25) (layer F.Cu) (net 1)))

